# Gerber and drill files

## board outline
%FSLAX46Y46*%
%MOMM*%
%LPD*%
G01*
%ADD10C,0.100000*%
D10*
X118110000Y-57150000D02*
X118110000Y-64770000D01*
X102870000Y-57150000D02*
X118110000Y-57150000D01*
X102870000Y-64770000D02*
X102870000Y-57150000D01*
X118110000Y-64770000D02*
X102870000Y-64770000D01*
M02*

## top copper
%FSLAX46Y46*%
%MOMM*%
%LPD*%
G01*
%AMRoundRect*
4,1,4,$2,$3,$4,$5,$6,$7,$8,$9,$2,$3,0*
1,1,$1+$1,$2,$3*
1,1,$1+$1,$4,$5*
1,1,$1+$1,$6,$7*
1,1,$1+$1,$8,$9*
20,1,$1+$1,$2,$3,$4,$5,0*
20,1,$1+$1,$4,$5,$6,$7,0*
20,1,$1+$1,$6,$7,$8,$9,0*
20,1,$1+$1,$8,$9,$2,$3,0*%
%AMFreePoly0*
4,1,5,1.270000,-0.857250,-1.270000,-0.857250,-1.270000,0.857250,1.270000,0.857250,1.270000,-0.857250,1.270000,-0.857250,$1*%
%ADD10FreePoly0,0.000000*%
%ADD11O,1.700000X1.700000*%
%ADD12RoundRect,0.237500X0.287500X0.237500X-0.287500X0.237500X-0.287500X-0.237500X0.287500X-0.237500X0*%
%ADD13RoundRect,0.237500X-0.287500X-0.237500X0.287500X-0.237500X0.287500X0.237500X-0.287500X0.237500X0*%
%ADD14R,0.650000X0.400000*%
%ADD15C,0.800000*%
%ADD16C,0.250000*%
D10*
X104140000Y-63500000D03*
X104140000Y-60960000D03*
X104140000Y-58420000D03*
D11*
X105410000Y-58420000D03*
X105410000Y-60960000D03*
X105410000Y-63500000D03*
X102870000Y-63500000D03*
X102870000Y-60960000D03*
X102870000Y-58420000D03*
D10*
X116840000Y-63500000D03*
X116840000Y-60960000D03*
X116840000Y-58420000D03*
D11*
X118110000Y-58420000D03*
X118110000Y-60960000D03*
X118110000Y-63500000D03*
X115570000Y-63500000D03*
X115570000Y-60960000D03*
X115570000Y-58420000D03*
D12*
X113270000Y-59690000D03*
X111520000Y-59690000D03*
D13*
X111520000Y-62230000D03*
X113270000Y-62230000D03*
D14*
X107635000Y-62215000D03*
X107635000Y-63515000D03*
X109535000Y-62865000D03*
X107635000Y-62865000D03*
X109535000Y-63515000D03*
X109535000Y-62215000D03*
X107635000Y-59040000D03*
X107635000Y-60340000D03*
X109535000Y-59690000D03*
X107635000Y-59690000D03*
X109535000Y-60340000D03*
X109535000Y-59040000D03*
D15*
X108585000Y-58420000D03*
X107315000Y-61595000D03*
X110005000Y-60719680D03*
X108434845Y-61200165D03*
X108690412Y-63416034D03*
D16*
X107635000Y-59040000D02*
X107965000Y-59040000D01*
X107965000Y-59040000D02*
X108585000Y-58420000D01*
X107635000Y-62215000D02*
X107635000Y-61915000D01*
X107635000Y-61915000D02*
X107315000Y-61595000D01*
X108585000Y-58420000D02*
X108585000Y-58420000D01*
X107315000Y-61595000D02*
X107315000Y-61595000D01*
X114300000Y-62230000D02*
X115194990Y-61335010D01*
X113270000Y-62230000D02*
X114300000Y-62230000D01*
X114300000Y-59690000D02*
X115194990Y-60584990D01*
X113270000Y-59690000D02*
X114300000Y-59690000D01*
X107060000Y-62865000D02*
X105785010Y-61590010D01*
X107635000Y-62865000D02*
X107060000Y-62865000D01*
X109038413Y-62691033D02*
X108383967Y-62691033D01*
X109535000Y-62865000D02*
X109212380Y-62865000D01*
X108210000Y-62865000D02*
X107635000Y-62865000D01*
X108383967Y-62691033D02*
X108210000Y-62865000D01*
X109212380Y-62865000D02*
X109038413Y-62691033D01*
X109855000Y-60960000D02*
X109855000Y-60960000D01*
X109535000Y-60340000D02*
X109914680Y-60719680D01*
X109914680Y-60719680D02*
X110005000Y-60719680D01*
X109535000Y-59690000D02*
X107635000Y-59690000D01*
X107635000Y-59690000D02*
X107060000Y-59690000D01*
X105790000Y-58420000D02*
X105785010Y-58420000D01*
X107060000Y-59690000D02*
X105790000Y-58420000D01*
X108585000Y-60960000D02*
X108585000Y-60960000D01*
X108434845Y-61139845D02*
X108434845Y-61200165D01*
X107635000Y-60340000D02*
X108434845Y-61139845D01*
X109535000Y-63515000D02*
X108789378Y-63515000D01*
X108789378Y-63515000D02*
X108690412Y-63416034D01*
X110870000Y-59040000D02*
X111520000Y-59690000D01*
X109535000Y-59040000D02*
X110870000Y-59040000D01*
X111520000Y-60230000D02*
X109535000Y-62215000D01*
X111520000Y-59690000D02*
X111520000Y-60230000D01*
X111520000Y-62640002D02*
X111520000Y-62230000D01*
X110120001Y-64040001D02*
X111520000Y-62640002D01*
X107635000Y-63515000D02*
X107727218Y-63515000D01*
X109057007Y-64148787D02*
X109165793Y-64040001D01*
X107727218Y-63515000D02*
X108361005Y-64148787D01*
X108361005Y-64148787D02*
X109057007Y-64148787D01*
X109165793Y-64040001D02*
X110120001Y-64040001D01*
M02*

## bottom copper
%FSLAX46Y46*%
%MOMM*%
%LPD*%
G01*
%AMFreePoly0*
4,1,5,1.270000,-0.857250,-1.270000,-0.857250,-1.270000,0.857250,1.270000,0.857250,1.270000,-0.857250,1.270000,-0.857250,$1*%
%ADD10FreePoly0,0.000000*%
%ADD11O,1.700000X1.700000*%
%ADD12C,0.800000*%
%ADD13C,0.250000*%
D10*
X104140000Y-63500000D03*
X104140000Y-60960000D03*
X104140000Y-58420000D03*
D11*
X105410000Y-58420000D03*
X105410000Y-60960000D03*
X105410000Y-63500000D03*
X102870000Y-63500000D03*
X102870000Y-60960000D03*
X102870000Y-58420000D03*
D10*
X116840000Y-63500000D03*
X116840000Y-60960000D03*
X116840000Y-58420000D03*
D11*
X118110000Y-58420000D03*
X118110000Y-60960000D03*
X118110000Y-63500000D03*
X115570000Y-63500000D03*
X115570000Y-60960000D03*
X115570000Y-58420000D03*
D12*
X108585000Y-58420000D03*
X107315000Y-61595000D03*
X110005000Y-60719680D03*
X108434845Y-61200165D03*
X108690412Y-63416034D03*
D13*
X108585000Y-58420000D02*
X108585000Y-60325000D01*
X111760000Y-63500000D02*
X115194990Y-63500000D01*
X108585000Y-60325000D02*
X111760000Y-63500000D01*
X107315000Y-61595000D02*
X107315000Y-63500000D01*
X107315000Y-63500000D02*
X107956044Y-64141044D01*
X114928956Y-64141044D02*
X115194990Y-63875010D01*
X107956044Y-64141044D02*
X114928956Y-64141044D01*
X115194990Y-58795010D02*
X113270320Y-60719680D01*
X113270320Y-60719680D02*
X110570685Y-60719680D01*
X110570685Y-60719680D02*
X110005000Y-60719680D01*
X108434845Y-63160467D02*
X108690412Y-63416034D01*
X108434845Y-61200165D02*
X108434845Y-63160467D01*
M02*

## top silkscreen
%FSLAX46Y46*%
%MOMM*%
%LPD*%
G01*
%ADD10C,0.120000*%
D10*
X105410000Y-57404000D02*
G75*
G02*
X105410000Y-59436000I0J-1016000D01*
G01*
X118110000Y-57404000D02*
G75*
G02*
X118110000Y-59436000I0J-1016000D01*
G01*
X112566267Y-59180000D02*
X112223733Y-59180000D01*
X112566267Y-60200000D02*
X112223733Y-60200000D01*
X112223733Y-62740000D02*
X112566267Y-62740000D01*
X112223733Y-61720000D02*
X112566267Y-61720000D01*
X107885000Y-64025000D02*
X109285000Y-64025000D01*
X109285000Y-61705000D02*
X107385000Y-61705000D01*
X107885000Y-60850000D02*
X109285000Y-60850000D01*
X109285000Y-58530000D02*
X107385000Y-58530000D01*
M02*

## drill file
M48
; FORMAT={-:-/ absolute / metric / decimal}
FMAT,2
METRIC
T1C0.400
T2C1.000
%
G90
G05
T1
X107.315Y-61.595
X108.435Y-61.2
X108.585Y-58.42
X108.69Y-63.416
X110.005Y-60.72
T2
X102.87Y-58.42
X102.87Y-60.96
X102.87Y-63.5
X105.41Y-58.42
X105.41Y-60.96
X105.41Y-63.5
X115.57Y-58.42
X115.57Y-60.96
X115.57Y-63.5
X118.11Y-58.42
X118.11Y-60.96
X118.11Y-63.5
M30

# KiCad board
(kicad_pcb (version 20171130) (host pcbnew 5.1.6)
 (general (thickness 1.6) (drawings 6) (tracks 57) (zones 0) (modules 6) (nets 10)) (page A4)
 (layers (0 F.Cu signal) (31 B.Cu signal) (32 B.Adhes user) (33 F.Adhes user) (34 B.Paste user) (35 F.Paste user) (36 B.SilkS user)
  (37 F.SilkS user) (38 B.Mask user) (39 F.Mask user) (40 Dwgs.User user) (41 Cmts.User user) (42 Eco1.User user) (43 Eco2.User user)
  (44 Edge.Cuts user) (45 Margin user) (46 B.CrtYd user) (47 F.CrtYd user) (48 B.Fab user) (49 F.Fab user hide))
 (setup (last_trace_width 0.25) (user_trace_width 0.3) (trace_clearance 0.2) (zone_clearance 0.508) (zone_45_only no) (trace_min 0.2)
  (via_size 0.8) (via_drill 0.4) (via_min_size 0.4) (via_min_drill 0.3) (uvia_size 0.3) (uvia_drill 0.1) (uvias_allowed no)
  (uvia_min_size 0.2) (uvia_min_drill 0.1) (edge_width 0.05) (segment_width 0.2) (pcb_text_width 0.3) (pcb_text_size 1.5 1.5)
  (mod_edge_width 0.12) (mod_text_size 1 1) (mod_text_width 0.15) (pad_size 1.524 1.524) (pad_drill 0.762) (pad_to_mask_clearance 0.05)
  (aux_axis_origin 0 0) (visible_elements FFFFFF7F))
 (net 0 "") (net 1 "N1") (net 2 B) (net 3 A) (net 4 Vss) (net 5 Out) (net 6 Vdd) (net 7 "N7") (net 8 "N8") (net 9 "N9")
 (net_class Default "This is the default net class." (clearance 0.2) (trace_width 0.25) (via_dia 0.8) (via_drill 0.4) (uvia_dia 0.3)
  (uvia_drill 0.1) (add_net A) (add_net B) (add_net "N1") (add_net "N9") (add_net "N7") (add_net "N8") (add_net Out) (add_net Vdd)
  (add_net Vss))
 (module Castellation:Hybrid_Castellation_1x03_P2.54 (layer F.Cu) (at 104.14 58.42)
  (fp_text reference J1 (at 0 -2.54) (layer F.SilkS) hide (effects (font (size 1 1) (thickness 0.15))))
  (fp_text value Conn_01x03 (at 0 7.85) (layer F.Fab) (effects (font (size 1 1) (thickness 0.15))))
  (fp_arc (start 1.27 0) (end 1.27 1.016) (angle -180) (layer F.SilkS) (width 0.12))
  (pad 3 connect custom (at 0 5.08) (size 2.54 1.7145) (layers B.Cu B.Mask) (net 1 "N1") (zone_connect 0)
   (options (clearance outline) (anchor rect)) (primitives))
  (pad 2 connect custom (at 0 2.54) (size 2.54 1.7145) (layers B.Cu B.Mask) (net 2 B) (zone_connect 0)
   (options (clearance outline) (anchor rect)) (primitives))
  (pad 1 connect custom (at 0 0) (size 2.54 1.7145) (layers B.Cu B.Mask) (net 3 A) (zone_connect 0)
   (options (clearance outline) (anchor rect)) (primitives))
  (pad 3 connect custom (at 0 5.08) (size 2.54 1.7145) (layers F.Cu F.Mask) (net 1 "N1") (zone_connect 0)
   (options (clearance outline) (anchor rect)) (primitives))
  (pad 2 connect custom (at 0 2.54) (size 2.54 1.7145) (layers F.Cu F.Mask) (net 2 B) (zone_connect 0)
   (options (clearance outline) (anchor rect)) (primitives))
  (pad 1 connect custom (at 0 0) (size 2.54 1.7145) (layers F.Cu F.Mask) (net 3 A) (zone_connect 0)
   (options (clearance outline) (anchor rect)) (primitives))
  (pad 1 thru_hole oval (at 1.27 0) (size 1.7 1.7) (drill 1) (layers *.Cu *.Mask) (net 3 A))
  (pad 2 thru_hole oval (at 1.27 2.54) (size 1.7 1.7) (drill 1) (layers *.Cu *.Mask) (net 2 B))
  (pad 3 thru_hole oval (at 1.27 5.08) (size 1.7 1.7) (drill 1) (layers *.Cu *.Mask) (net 1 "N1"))
  (pad 3 thru_hole oval (at -1.27 5.08) (size 1.7 1.7) (drill 1) (layers *.Cu *.Mask) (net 1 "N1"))
  (pad 2 thru_hole oval (at -1.27 2.54) (size 1.7 1.7) (drill 1) (layers *.Cu *.Mask) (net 2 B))
  (pad 1 thru_hole oval (at -1.27 0) (size 1.7 1.7) (drill 1) (layers *.Cu *.Mask) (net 3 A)))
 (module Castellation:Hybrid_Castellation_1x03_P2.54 (layer F.Cu) (at 116.84 58.42)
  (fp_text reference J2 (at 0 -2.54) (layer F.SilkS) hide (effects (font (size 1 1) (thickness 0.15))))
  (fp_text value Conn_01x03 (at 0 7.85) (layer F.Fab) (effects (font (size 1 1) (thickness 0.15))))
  (fp_arc (start 1.27 0) (end 1.27 1.016) (angle -180) (layer F.SilkS) (width 0.12))
  (pad 3 connect custom (at 0 5.08) (size 2.54 1.7145) (layers B.Cu B.Mask) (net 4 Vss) (zone_connect 0)
   (options (clearance outline) (anchor rect)) (primitives))
  (pad 2 connect custom (at 0 2.54) (size 2.54 1.7145) (layers B.Cu B.Mask) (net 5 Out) (zone_connect 0)
   (options (clearance outline) (anchor rect)) (primitives))
  (pad 1 connect custom (at 0 0) (size 2.54 1.7145) (layers B.Cu B.Mask) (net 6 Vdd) (zone_connect 0)
   (options (clearance outline) (anchor rect)) (primitives))
  (pad 3 connect custom (at 0 5.08) (size 2.54 1.7145) (layers F.Cu F.Mask) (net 4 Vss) (zone_connect 0)
   (options (clearance outline) (anchor rect)) (primitives))
  (pad 2 connect custom (at 0 2.54) (size 2.54 1.7145) (layers F.Cu F.Mask) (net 5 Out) (zone_connect 0)
   (options (clearance outline) (anchor rect)) (primitives))
  (pad 1 connect custom (at 0 0) (size 2.54 1.7145) (layers F.Cu F.Mask) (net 6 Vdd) (zone_connect 0)
   (options (clearance outline) (anchor rect)) (primitives))
  (pad 1 thru_hole oval (at 1.27 0) (size 1.7 1.7) (drill 1) (layers *.Cu *.Mask) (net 6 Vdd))
  (pad 2 thru_hole oval (at 1.27 2.54) (size 1.7 1.7) (drill 1) (layers *.Cu *.Mask) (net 5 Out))
  (pad 3 thru_hole oval (at 1.27 5.08) (size 1.7 1.7) (drill 1) (layers *.Cu *.Mask) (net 4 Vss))
  (pad 3 thru_hole oval (at -1.27 5.08) (size 1.7 1.7) (drill 1) (layers *.Cu *.Mask) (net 4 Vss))
  (pad 2 thru_hole oval (at -1.27 2.54) (size 1.7 1.7) (drill 1) (layers *.Cu *.Mask) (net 5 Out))
  (pad 1 thru_hole oval (at -1.27 0) (size 1.7 1.7) (drill 1) (layers *.Cu *.Mask) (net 6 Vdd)))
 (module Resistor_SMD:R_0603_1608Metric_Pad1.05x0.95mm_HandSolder (layer F.Cu) (at 112.395 59.69 180)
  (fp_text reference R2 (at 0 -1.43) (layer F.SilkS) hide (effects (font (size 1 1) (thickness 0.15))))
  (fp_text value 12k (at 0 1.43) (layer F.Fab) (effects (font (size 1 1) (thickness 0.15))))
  (fp_line (start -0.171267 0.51) (end 0.171267 0.51) (layer F.SilkS) (width 0.12))
  (fp_line (start -0.171267 -0.51) (end 0.171267 -0.51) (layer F.SilkS) (width 0.12))
  (pad 1 smd roundrect (at -0.875 0 180) (size 1.05 0.95) (layers F.Cu F.Paste F.Mask) (roundrect_rratio 0.25) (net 5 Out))
  (pad 2 smd roundrect (at 0.875 0 180) (size 1.05 0.95) (layers F.Cu F.Paste F.Mask) (roundrect_rratio 0.25) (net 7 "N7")))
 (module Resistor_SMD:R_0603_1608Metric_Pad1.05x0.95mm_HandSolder (layer F.Cu) (at 112.395 62.23)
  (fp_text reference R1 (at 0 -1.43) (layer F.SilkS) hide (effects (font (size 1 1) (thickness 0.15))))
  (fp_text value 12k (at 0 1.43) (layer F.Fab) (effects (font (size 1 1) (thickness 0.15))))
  (fp_line (start -0.171267 0.51) (end 0.171267 0.51) (layer F.SilkS) (width 0.12))
  (fp_line (start -0.171267 -0.51) (end 0.171267 -0.51) (layer F.SilkS) (width 0.12))
  (pad 1 smd roundrect (at -0.875 0) (size 1.05 0.95) (layers F.Cu F.Paste F.Mask) (roundrect_rratio 0.25) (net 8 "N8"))
  (pad 2 smd roundrect (at 0.875 0) (size 1.05 0.95) (layers F.Cu F.Paste F.Mask) (roundrect_rratio 0.25) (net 5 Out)))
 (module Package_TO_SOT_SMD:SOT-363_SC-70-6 (layer F.Cu) (at 108.585 62.865)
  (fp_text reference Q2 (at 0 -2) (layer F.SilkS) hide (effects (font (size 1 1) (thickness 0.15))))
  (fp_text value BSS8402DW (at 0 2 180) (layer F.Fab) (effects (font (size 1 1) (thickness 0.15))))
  (fp_line (start -0.7 1.16) (end 0.7 1.16) (layer F.SilkS) (width 0.12))
  (fp_line (start 0.7 -1.16) (end -1.2 -1.16) (layer F.SilkS) (width 0.12))
  (pad 1 smd rect (at -0.95 -0.65) (size 0.65 0.4) (layers F.Cu F.Paste F.Mask) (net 4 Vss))
  (pad 3 smd rect (at -0.95 0.65) (size 0.65 0.4) (layers F.Cu F.Paste F.Mask) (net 8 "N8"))
  (pad 5 smd rect (at 0.95 0) (size 0.65 0.4) (layers F.Cu F.Paste F.Mask) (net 2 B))
  (pad 2 smd rect (at -0.95 0) (size 0.65 0.4) (layers F.Cu F.Paste F.Mask) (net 2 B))
  (pad 4 smd rect (at 0.95 0.65) (size 0.65 0.4) (layers F.Cu F.Paste F.Mask) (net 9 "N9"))
  (pad 6 smd rect (at 0.95 -0.65) (size 0.65 0.4) (layers F.Cu F.Paste F.Mask) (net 7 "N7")))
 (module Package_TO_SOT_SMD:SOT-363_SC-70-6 (layer F.Cu) (at 108.585 59.69)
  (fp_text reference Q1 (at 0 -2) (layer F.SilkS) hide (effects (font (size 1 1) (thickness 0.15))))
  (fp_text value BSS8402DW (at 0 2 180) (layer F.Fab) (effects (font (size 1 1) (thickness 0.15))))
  (fp_line (start -0.7 1.16) (end 0.7 1.16) (layer F.SilkS) (width 0.12))
  (fp_line (start 0.7 -1.16) (end -1.2 -1.16) (layer F.SilkS) (width 0.12))
  (pad 1 smd rect (at -0.95 -0.65) (size 0.65 0.4) (layers F.Cu F.Paste F.Mask) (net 4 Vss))
  (pad 3 smd rect (at -0.95 0.65) (size 0.65 0.4) (layers F.Cu F.Paste F.Mask) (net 9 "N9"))
  (pad 5 smd rect (at 0.95 0) (size 0.65 0.4) (layers F.Cu F.Paste F.Mask) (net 3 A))
  (pad 2 smd rect (at -0.95 0) (size 0.65 0.4) (layers F.Cu F.Paste F.Mask) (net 3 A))
  (pad 4 smd rect (at 0.95 0.65) (size 0.65 0.4) (layers F.Cu F.Paste F.Mask) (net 6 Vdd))
  (pad 6 smd rect (at 0.95 -0.65) (size 0.65 0.4) (layers F.Cu F.Paste F.Mask) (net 7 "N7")))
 (gr_line (start 118.11 57.15) (end 118.11 64.77) (layer Edge.Cuts) (width 0.1))
 (gr_line (start 102.87 57.15) (end 118.11 57.15) (layer Edge.Cuts) (width 0.1))
 (gr_line (start 102.87 64.77) (end 102.87 57.15) (layer Edge.Cuts) (width 0.1))
 (gr_line (start 118.11 64.77) (end 102.87 64.77) (layer Edge.Cuts) (width 0.1))
 (segment (start 107.635 59.04) (end 107.965 59.04) (width 0.25) (layer F.Cu) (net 4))
 (segment (start 107.965 59.04) (end 108.585 58.42) (width 0.25) (layer F.Cu) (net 4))
 (segment (start 107.635 62.215) (end 107.635 61.915) (width 0.25) (layer F.Cu) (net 4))
 (segment (start 107.635 61.915) (end 107.315 61.595) (width 0.25) (layer F.Cu) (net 4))
 (segment (start 108.585 58.42) (end 108.585 58.42) (width 0.25) (layer F.Cu) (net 4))
 (via (at 108.585 58.42) (size 0.8) (drill 0.4) (layers F.Cu B.Cu) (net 4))
 (segment (start 107.315 61.595) (end 107.315 61.595) (width 0.25) (layer F.Cu) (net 4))
 (via (at 107.315 61.595) (size 0.8) (drill 0.4) (layers F.Cu B.Cu) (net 4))
 (segment (start 108.585 58.42) (end 108.585 60.325) (width 0.25) (layer B.Cu) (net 4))
 (segment (start 111.76 63.5) (end 115.19499 63.5) (width 0.25) (layer B.Cu) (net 4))
 (segment (start 108.585 60.325) (end 111.76 63.5) (width 0.25) (layer B.Cu) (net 4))
 (segment (start 107.315 61.595) (end 107.315 63.5) (width 0.25) (layer B.Cu) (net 4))
 (segment (start 107.315 63.5) (end 107.956044 64.141044) (width 0.25) (layer B.Cu) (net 4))
 (segment (start 114.928956 64.141044) (end 115.19499 63.87501) (width 0.25) (layer B.Cu) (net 4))
 (segment (start 107.956044 64.141044) (end 114.928956 64.141044) (width 0.25) (layer B.Cu) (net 4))
 (segment (start 114.3 62.23) (end 115.19499 61.33501) (width 0.25) (layer F.Cu) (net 5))
 (segment (start 113.27 62.23) (end 114.3 62.23) (width 0.25) (layer F.Cu) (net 5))
 (segment (start 114.3 59.69) (end 115.19499 60.58499) (width 0.25) (layer F.Cu) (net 5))
 (segment (start 113.27 59.69) (end 114.3 59.69) (width 0.25) (layer F.Cu) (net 5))
 (segment (start 107.06 62.865) (end 105.78501 61.59001) (width 0.25) (layer F.Cu) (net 2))
 (segment (start 107.635 62.865) (end 107.06 62.865) (width 0.25) (layer F.Cu) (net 2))
 (segment (start 109.038413 62.691033) (end 108.383967 62.691033) (width 0.25) (layer F.Cu) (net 2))
 (segment (start 109.535 62.865) (end 109.21238 62.865) (width 0.25) (layer F.Cu) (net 2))
 (segment (start 108.21 62.865) (end 107.635 62.865) (width 0.25) (layer F.Cu) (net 2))
 (segment (start 108.383967 62.691033) (end 108.21 62.865) (width 0.25) (layer F.Cu) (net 2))
 (segment (start 109.21238 62.865) (end 109.038413 62.691033) (width 0.25) (layer F.Cu) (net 2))
 (segment (start 109.855 60.96) (end 109.855 60.96) (width 0.25) (layer F.Cu) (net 6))
 (via (at 110.005 60.71968) (size 0.8) (drill 0.4) (layers F.Cu B.Cu) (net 6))
 (segment (start 109.535 60.34) (end 109.91468 60.71968) (width 0.25) (layer F.Cu) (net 6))
 (segment (start 115.19499 58.79501) (end 113.27032 60.71968) (width 0.25) (layer B.Cu) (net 6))
 (segment (start 113.27032 60.71968) (end 110.570685 60.71968) (width 0.25) (layer B.Cu) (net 6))
 (segment (start 110.570685 60.71968) (end 110.005 60.71968) (width 0.25) (layer B.Cu) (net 6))
 (segment (start 109.91468 60.71968) (end 110.005 60.71968) (width 0.25) (layer F.Cu) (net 6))
 (segment (start 109.535 59.69) (end 107.635 59.69) (width 0.25) (layer F.Cu) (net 3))
 (segment (start 107.635 59.69) (end 107.06 59.69) (width 0.25) (layer F.Cu) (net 3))
 (segment (start 105.79 58.42) (end 105.78501 58.42) (width 0.25) (layer F.Cu) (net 3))
 (segment (start 107.06 59.69) (end 105.79 58.42) (width 0.25) (layer F.Cu) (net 3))
 (segment (start 108.585 60.96) (end 108.585 60.96) (width 0.25) (layer F.Cu) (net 9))
 (via (at 108.434845 61.200165) (size 0.8) (drill 0.4) (layers F.Cu B.Cu) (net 9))
 (segment (start 108.434845 61.139845) (end 108.434845 61.200165) (width 0.25) (layer F.Cu) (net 9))
 (segment (start 107.635 60.34) (end 108.434845 61.139845) (width 0.25) (layer F.Cu) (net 9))
 (segment (start 108.434845 63.160467) (end 108.690412 63.416034) (width 0.25) (layer B.Cu) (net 9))
 (segment (start 108.434845 61.200165) (end 108.434845 63.160467) (width 0.25) (layer B.Cu) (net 9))
 (segment (start 109.535 63.515) (end 108.789378 63.515) (width 0.25) (layer F.Cu) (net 9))
 (segment (start 108.789378 63.515) (end 108.690412 63.416034) (width 0.25) (layer F.Cu) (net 9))
 (via (at 108.690412 63.416034) (size 0.8) (drill 0.4) (layers F.Cu B.Cu) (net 9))
 (segment (start 110.87 59.04) (end 111.52 59.69) (width 0.25) (layer F.Cu) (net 7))
 (segment (start 109.535 59.04) (end 110.87 59.04) (width 0.25) (layer F.Cu) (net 7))
 (segment (start 111.52 60.23) (end 109.535 62.215) (width 0.25) (layer F.Cu) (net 7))
 (segment (start 111.52 59.69) (end 111.52 60.23) (width 0.25) (layer F.Cu) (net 7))
 (segment (start 111.52 62.640002) (end 111.52 62.23) (width 0.25) (layer F.Cu) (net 8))
 (segment (start 110.120001 64.040001) (end 111.52 62.640002) (width 0.25) (layer F.Cu) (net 8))
 (segment (start 107.635 63.515) (end 107.727218 63.515) (width 0.25) (layer F.Cu) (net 8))
 (segment (start 109.057007 64.148787) (end 109.165793 64.040001) (width 0.25) (layer F.Cu) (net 8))
 (segment (start 107.727218 63.515) (end 108.361005 64.148787) (width 0.25) (layer F.Cu) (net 8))
 (segment (start 108.361005 64.148787) (end 109.057007 64.148787) (width 0.25) (layer F.Cu) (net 8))
 (segment (start 109.165793 64.040001) (end 110.120001 64.040001) (width 0.25) (layer F.Cu) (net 8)))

